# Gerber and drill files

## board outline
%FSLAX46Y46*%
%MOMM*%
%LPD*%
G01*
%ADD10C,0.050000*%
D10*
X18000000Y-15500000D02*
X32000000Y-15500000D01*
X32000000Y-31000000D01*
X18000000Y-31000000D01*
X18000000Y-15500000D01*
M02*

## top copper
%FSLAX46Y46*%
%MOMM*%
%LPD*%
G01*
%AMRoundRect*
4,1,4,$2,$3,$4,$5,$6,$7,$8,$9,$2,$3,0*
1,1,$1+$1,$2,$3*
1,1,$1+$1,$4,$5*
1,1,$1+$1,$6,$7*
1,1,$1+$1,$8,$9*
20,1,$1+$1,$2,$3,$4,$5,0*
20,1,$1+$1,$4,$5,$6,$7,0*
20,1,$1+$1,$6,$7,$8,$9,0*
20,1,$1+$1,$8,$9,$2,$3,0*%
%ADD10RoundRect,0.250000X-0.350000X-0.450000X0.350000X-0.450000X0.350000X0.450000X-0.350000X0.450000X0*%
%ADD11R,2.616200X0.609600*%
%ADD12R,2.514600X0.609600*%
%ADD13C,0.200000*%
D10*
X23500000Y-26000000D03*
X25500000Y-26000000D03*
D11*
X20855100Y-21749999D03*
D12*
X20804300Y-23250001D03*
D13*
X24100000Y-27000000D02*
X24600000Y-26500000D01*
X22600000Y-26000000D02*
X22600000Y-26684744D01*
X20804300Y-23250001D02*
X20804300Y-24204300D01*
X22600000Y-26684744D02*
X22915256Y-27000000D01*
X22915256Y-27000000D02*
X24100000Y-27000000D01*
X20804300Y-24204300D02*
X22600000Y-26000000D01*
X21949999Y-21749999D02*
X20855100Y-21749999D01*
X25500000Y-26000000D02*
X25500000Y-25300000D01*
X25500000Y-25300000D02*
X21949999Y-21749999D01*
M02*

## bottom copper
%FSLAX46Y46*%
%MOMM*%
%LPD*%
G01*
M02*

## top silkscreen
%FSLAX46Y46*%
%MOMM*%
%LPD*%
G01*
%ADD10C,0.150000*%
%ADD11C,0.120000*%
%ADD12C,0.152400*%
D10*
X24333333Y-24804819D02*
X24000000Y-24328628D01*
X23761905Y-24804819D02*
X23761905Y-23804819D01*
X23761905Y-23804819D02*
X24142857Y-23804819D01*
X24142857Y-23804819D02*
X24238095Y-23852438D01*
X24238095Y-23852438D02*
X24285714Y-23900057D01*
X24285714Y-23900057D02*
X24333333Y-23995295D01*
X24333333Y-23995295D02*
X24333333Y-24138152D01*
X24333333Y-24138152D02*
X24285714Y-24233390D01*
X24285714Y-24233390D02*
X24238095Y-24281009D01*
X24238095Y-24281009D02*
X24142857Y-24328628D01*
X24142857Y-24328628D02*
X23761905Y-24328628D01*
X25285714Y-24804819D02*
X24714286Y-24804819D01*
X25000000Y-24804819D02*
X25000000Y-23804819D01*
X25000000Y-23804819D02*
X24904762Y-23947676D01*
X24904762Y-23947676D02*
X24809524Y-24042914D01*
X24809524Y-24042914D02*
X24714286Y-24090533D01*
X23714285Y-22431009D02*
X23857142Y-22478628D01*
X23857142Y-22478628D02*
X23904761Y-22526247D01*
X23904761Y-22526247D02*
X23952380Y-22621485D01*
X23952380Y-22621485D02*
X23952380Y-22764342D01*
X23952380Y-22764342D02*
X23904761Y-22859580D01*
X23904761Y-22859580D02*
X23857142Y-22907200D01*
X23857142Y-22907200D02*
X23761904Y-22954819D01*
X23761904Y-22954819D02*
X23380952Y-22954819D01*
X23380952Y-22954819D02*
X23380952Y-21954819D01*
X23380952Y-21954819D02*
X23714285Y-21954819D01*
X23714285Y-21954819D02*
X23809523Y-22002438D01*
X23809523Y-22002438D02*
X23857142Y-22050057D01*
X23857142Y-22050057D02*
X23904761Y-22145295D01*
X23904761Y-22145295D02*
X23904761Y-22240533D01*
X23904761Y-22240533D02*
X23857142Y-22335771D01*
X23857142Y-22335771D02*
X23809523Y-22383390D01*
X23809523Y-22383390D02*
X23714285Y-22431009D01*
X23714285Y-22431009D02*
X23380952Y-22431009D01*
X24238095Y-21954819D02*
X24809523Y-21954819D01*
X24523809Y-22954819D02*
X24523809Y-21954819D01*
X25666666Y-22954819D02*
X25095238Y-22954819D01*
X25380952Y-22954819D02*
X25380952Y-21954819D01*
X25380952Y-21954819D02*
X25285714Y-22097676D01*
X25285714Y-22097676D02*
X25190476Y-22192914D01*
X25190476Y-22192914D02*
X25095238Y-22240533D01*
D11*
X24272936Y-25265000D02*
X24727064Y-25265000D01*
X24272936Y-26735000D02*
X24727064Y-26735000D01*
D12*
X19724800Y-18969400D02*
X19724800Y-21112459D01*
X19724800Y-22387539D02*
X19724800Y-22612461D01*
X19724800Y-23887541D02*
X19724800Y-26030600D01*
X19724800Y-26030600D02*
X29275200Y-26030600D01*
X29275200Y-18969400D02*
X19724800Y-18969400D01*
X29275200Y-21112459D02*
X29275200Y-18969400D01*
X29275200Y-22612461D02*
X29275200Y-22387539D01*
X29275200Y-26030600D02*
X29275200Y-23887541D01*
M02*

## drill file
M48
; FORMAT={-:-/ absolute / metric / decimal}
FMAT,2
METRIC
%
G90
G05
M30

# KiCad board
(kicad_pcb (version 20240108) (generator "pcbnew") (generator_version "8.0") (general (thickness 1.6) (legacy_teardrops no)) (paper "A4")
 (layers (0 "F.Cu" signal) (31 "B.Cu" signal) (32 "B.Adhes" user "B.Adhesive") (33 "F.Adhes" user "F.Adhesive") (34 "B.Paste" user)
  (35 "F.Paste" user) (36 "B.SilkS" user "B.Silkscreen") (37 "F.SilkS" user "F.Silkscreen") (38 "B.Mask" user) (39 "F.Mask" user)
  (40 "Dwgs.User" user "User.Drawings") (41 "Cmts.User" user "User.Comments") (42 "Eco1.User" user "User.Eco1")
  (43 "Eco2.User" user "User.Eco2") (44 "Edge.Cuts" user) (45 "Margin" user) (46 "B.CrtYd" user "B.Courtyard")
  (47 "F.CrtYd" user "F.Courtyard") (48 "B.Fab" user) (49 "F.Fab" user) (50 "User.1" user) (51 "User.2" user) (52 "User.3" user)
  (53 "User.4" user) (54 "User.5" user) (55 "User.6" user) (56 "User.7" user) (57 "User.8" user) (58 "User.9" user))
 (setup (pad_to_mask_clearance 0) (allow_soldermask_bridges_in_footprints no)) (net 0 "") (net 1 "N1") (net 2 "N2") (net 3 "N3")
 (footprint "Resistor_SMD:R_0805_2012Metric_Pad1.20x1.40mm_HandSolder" (layer "F.Cu") (at 24.5 26)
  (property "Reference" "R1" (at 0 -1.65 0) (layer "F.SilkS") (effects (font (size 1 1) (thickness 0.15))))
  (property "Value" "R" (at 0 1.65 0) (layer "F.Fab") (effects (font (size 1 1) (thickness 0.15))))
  (fp_line (start -0.227064 -0.735) (end 0.227064 -0.735) (stroke (width 0.12) (type solid)) (layer "F.SilkS"))
  (fp_line (start -0.227064 0.735) (end 0.227064 0.735) (stroke (width 0.12) (type solid)) (layer "F.SilkS"))
  (pad "1" smd roundrect (at -1 0) (size 1.2 1.4) (layers "F.Cu" "F.Paste" "F.Mask") (roundrect_rratio 0.208333) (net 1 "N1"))
  (pad "2" smd roundrect (at 1 0) (size 1.2 1.4) (layers "F.Cu" "F.Paste" "F.Mask") (roundrect_rratio 0.208333) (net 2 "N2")))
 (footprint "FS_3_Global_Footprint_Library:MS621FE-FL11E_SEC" (layer "F.Cu") (at 24.5 22.5)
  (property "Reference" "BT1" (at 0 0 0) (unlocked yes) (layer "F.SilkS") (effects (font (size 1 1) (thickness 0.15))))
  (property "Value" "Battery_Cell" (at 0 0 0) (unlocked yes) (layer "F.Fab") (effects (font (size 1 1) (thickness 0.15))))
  (fp_line (start -4.7752 -3.5306) (end -4.7752 -1.387541) (stroke (width 0.1524) (type solid)) (layer "F.SilkS"))
  (fp_line (start -4.7752 -0.112461) (end -4.7752 0.112461) (stroke (width 0.1524) (type solid)) (layer "F.SilkS"))
  (fp_line (start -4.7752 1.387541) (end -4.7752 3.5306) (stroke (width 0.1524) (type solid)) (layer "F.SilkS"))
  (fp_line (start -4.7752 3.5306) (end 4.7752 3.5306) (stroke (width 0.1524) (type solid)) (layer "F.SilkS"))
  (fp_line (start 4.7752 -3.5306) (end -4.7752 -3.5306) (stroke (width 0.1524) (type solid)) (layer "F.SilkS"))
  (fp_line (start 4.7752 -1.387541) (end 4.7752 -3.5306) (stroke (width 0.1524) (type solid)) (layer "F.SilkS"))
  (fp_line (start 4.7752 0.112461) (end 4.7752 -0.112461) (stroke (width 0.1524) (type solid)) (layer "F.SilkS"))
  (fp_line (start 4.7752 3.5306) (end 4.7752 1.387541) (stroke (width 0.1524) (type solid)) (layer "F.SilkS"))
  (pad "1" smd rect (at -3.6449 -0.750001) (size 2.6162 0.6096) (layers "F.Cu" "F.Paste" "F.Mask") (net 2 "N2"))
  (pad "2" smd rect (at -3.6957 0.750001) (size 2.5146 0.6096) (layers "F.Cu" "F.Paste" "F.Mask") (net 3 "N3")))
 (gr_rect (start 18 15.5) (end 32 31) (stroke (width 0.05) (type default)) (fill none) (layer "Edge.Cuts"))
 (segment (start 24.1 27) (end 24.6 26.5) (width 0.2) (layer "F.Cu") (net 3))
 (segment (start 22.6 26) (end 22.6 26.684744) (width 0.2) (layer "F.Cu") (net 3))
 (segment (start 20.8043 23.250001) (end 20.8043 24.2043) (width 0.2) (layer "F.Cu") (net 3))
 (segment (start 22.6 26.684744) (end 22.915256 27) (width 0.2) (layer "F.Cu") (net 3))
 (segment (start 22.915256 27) (end 24.1 27) (width 0.2) (layer "F.Cu") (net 3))
 (segment (start 20.8043 24.2043) (end 22.6 26) (width 0.2) (layer "F.Cu") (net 3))
 (segment (start 21.949999 21.749999) (end 20.8551 21.749999) (width 0.2) (layer "F.Cu") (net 2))
 (segment (start 25.5 26) (end 25.5 25.3) (width 0.2) (layer "F.Cu") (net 2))
 (segment (start 25.5 25.3) (end 21.949999 21.749999) (width 0.2) (layer "F.Cu") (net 2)))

